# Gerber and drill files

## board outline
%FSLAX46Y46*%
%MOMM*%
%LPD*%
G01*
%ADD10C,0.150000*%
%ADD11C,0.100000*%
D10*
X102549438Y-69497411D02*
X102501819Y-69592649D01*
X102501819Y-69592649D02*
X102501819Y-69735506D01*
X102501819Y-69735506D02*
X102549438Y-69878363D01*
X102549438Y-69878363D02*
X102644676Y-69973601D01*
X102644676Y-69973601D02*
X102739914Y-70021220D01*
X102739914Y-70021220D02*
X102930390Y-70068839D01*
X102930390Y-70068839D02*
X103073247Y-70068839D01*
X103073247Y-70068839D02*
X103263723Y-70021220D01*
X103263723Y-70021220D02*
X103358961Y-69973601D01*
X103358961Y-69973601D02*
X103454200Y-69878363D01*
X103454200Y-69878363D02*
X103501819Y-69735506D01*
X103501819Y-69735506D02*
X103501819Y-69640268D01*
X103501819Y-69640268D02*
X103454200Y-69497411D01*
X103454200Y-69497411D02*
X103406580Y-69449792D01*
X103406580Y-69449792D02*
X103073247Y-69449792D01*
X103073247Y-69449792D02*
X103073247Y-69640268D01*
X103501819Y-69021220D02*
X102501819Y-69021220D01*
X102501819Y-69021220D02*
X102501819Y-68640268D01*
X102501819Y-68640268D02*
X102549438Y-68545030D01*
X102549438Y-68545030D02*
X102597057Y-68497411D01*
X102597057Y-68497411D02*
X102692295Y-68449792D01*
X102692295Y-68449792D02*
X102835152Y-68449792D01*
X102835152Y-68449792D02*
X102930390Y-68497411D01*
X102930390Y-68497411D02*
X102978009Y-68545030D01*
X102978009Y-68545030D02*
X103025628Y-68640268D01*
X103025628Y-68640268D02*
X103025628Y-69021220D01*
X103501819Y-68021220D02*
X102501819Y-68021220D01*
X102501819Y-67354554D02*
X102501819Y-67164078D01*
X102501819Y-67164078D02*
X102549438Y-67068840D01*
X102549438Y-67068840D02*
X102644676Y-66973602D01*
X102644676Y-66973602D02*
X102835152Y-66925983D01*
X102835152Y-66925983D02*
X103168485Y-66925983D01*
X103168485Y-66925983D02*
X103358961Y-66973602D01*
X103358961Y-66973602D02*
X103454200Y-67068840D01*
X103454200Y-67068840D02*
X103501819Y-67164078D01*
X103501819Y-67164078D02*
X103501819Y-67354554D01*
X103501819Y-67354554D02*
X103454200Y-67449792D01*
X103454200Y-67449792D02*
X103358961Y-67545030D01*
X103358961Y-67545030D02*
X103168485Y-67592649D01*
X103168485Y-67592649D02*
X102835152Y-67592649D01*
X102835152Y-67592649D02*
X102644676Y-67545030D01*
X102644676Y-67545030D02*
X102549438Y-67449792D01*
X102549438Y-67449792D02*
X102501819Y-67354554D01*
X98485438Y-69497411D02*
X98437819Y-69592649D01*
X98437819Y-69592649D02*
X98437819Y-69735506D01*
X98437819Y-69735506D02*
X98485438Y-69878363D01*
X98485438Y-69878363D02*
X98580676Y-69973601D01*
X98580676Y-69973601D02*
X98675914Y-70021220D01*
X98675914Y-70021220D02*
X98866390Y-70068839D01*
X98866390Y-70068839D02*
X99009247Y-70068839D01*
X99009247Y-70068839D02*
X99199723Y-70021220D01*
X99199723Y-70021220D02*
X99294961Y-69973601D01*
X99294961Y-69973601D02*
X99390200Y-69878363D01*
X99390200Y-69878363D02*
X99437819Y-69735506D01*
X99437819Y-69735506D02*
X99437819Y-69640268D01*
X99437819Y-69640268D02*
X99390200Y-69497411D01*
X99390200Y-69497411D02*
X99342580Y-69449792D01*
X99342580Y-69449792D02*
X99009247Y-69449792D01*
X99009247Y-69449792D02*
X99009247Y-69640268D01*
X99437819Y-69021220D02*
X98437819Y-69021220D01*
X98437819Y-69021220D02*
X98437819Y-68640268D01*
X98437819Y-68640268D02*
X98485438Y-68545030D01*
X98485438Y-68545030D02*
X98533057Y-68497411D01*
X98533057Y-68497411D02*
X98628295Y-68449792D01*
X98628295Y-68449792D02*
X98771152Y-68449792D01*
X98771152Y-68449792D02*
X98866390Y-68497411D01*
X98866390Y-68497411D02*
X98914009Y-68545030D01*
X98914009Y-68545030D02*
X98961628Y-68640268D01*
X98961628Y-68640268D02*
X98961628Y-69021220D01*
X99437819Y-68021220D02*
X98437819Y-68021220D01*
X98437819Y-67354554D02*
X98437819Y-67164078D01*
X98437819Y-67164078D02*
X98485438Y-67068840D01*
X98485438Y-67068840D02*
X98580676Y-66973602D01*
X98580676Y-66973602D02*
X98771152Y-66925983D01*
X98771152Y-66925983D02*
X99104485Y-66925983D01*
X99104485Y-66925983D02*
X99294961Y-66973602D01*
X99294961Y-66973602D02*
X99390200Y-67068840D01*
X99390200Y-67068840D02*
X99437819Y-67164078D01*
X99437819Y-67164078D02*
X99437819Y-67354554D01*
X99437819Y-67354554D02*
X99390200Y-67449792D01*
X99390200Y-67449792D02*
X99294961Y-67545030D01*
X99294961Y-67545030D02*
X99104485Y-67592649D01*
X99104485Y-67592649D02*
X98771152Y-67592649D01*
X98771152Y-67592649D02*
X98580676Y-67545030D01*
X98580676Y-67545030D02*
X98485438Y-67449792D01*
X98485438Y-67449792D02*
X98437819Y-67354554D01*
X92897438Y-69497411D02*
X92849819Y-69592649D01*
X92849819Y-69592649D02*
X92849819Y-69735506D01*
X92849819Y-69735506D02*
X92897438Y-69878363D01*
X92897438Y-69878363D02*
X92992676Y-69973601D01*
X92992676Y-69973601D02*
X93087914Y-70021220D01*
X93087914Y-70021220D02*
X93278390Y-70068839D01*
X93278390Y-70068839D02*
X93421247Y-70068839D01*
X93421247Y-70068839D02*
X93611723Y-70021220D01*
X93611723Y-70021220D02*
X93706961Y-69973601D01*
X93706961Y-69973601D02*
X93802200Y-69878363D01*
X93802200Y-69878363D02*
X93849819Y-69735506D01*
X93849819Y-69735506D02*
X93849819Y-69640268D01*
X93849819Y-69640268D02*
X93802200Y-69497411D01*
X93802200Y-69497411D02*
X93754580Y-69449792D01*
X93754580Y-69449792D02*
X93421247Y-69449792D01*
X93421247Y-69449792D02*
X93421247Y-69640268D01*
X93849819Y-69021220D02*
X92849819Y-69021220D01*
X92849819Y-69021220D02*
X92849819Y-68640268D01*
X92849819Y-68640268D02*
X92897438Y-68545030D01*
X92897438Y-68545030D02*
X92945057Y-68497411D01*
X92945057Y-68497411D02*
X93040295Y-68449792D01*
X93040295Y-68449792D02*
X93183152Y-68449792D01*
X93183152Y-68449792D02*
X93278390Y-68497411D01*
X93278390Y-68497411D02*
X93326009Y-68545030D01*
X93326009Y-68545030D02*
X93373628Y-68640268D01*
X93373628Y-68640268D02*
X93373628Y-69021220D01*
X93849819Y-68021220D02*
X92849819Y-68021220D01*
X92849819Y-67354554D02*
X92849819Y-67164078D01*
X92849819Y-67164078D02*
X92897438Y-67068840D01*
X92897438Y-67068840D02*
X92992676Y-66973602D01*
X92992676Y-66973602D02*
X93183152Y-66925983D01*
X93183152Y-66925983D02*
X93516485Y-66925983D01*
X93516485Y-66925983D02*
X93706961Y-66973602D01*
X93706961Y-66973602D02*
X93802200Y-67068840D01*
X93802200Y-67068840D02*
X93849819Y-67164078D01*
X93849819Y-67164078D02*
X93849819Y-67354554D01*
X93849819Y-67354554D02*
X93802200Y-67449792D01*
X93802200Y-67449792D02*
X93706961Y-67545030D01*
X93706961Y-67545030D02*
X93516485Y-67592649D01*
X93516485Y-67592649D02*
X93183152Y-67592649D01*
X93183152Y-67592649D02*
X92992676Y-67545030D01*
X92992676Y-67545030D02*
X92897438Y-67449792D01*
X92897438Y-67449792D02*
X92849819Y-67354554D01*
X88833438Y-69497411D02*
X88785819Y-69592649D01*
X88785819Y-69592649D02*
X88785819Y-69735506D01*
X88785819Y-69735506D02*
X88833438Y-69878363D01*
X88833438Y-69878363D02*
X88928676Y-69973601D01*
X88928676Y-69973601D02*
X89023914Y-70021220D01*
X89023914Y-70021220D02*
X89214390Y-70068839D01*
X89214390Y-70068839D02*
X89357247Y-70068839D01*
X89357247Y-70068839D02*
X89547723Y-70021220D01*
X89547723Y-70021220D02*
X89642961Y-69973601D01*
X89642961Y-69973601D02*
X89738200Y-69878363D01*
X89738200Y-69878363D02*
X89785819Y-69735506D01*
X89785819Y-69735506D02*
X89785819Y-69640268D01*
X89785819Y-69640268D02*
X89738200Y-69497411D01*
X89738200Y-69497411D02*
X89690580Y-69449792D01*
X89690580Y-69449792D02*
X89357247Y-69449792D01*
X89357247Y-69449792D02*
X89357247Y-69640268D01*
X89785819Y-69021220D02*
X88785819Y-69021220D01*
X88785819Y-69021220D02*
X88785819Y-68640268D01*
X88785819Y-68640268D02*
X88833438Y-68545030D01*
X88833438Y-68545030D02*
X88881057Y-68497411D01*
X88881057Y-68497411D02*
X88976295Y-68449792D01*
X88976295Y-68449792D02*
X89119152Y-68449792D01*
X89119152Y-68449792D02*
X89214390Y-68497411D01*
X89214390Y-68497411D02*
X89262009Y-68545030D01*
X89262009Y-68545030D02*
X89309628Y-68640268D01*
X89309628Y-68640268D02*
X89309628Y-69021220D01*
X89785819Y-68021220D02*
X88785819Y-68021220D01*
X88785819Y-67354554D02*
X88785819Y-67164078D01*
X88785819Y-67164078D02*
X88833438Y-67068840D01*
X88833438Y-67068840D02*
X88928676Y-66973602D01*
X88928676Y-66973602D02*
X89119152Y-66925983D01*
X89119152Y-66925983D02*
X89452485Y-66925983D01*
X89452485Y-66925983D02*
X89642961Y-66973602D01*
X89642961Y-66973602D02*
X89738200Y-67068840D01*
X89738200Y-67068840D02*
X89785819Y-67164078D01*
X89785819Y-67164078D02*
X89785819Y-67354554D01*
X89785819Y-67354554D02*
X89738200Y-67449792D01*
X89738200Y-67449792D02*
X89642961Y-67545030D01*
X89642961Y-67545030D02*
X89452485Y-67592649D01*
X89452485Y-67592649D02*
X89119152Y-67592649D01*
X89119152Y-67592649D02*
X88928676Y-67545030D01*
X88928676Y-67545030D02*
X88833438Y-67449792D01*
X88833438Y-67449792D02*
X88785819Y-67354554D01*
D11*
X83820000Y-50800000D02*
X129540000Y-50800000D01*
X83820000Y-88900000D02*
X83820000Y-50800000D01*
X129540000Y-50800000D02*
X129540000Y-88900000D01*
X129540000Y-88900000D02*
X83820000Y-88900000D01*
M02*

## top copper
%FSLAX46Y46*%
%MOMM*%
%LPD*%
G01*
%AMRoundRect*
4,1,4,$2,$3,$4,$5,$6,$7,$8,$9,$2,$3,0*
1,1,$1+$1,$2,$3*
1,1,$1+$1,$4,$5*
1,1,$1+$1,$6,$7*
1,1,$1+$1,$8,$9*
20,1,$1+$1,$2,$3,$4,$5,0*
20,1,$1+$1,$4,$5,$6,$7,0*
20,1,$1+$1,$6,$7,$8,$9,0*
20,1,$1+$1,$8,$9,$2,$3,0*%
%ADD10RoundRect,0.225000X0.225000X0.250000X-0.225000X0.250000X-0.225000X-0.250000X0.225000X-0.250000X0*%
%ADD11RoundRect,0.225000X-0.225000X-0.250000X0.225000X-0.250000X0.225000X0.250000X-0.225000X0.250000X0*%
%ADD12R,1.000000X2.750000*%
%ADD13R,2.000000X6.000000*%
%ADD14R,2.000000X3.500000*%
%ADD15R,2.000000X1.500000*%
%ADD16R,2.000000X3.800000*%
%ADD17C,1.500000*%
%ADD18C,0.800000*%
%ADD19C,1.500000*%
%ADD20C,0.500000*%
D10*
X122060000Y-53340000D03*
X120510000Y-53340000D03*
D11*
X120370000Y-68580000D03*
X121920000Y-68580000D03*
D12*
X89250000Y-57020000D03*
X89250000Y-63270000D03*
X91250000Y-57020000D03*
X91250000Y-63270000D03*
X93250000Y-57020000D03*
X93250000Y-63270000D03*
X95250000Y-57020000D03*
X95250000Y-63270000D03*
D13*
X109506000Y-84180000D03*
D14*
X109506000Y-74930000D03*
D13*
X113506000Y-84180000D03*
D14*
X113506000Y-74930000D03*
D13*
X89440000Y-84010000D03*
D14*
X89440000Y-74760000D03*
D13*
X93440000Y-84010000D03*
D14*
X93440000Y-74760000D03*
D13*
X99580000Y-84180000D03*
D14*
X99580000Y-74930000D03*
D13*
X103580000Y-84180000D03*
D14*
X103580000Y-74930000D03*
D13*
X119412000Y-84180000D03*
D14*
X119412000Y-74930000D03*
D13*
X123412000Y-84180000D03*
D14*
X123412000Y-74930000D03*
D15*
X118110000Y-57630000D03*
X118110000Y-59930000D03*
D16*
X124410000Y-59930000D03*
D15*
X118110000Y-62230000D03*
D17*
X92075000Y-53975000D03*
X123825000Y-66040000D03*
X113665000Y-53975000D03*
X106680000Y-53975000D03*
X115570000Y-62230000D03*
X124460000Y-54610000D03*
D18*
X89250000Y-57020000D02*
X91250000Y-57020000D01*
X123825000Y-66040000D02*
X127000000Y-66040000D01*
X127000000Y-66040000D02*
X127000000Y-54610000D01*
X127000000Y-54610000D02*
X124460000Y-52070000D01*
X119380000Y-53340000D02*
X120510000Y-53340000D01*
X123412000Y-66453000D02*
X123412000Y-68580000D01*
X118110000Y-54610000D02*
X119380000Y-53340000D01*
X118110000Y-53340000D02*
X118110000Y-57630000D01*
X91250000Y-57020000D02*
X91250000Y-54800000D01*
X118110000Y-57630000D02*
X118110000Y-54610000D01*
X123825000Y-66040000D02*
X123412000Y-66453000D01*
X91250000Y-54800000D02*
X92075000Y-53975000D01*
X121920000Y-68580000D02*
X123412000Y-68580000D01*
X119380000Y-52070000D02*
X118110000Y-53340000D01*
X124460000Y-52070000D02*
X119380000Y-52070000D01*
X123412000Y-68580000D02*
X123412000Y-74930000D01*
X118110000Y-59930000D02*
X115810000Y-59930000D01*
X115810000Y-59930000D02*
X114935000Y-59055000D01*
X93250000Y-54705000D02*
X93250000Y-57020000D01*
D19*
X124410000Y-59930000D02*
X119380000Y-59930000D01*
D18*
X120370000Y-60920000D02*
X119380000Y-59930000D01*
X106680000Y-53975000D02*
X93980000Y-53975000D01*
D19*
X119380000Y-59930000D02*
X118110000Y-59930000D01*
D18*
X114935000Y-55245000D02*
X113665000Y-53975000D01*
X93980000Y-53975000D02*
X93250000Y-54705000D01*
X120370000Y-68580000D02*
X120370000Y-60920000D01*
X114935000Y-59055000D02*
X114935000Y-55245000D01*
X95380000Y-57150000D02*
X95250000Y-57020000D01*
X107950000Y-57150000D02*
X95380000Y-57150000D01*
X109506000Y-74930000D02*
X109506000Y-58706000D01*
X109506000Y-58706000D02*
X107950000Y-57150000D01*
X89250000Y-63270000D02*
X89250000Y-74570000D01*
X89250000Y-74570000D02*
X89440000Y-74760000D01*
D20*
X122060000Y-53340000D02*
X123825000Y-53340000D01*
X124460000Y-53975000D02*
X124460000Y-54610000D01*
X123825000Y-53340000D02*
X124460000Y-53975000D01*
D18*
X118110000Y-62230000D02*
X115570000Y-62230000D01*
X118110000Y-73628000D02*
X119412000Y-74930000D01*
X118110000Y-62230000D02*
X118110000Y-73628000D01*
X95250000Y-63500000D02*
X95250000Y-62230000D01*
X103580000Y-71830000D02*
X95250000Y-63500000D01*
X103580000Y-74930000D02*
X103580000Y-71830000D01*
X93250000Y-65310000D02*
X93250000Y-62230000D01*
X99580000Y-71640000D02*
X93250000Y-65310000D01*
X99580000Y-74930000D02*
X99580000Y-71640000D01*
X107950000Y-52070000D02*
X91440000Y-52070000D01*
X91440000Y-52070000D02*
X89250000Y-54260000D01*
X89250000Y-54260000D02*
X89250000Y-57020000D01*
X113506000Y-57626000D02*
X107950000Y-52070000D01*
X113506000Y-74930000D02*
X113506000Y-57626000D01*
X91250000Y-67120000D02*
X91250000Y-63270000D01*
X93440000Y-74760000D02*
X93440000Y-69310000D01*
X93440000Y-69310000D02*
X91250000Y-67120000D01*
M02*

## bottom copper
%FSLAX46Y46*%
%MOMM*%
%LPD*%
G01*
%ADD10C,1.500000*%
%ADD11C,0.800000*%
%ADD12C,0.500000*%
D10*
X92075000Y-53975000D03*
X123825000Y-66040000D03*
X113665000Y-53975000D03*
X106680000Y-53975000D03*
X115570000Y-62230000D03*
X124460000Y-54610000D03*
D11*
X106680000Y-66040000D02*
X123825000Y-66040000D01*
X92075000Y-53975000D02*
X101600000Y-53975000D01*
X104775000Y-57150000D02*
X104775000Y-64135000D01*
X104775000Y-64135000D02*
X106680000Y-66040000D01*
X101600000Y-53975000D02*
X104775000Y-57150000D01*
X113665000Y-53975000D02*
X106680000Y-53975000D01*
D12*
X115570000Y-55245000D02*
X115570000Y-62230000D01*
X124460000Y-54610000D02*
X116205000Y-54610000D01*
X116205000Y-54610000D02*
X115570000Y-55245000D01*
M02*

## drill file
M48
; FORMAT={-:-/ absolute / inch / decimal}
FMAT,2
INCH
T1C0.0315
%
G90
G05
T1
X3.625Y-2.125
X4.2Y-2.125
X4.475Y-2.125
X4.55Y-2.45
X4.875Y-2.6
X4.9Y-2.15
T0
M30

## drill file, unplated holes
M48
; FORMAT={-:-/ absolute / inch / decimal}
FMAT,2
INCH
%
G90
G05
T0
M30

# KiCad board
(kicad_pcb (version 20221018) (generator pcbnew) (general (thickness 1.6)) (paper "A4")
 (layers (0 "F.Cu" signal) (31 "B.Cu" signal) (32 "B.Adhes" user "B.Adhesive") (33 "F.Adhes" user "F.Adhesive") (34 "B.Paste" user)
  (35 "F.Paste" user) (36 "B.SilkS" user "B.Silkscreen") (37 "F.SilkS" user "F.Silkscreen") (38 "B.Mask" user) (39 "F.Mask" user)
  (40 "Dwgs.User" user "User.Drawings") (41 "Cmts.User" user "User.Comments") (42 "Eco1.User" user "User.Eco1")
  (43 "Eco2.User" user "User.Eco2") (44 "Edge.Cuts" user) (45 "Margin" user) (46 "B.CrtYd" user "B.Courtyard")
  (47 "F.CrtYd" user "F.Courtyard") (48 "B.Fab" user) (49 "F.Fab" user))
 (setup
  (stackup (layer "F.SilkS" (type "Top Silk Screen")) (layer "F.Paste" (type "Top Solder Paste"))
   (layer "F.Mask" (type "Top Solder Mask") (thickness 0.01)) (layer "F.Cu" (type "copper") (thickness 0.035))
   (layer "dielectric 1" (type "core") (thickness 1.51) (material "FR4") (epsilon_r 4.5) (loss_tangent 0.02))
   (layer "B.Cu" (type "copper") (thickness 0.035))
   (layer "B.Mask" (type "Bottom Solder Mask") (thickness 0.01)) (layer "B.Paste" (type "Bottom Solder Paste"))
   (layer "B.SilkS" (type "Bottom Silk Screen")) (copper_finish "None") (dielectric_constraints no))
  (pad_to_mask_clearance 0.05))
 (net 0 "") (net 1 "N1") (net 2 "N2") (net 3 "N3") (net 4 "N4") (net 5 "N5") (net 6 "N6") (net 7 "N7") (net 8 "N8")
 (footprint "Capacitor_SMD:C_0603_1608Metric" (layer "F.Cu") (at 121.285 53.34 180)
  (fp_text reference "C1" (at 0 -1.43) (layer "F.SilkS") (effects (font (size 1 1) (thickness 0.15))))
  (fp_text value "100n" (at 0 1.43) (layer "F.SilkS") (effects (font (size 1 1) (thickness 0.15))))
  (pad "1" smd roundrect (at -0.775 0 180) (size 0.9 0.95) (layers "F.Cu" "F.Paste" "F.Mask") (roundrect_rratio 0.25) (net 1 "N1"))
  (pad "2" smd roundrect (at 0.775 0 180) (size 0.9 0.95) (layers "F.Cu" "F.Paste" "F.Mask") (roundrect_rratio 0.25) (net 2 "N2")))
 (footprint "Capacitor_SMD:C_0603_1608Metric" (layer "F.Cu") (at 121.145 68.58)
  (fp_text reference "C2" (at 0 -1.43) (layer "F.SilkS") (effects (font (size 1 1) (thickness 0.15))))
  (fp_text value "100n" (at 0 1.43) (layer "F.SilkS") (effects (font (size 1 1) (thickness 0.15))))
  (pad "1" smd roundrect (at -0.775 0) (size 0.9 0.95) (layers "F.Cu" "F.Paste" "F.Mask") (roundrect_rratio 0.25) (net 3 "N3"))
  (pad "2" smd roundrect (at 0.775 0) (size 0.9 0.95) (layers "F.Cu" "F.Paste" "F.Mask") (roundrect_rratio 0.25) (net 2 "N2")))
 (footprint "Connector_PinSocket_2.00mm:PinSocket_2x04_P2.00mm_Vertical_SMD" (layer "F.Cu") (at 92.25 60.145 90)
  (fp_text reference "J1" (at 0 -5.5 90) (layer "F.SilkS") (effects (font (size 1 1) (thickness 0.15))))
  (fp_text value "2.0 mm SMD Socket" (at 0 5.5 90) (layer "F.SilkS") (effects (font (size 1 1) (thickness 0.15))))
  (pad "1" smd rect (at 3.125 -3 90) (size 2.75 1) (layers "F.Cu" "F.Paste" "F.Mask") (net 2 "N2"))
  (pad "2" smd rect (at -3.125 -3 90) (size 2.75 1) (layers "F.Cu" "F.Paste" "F.Mask") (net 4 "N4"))
  (pad "3" smd rect (at 3.125 -1 90) (size 2.75 1) (layers "F.Cu" "F.Paste" "F.Mask") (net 2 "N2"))
  (pad "4" smd rect (at -3.125 -1 90) (size 2.75 1) (layers "F.Cu" "F.Paste" "F.Mask") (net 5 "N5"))
  (pad "5" smd rect (at 3.125 1 90) (size 2.75 1) (layers "F.Cu" "F.Paste" "F.Mask") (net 3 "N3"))
  (pad "6" smd rect (at -3.125 1 90) (size 2.75 1) (layers "F.Cu" "F.Paste" "F.Mask") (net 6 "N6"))
  (pad "7" smd rect (at 3.125 3 90) (size 2.75 1) (layers "F.Cu" "F.Paste" "F.Mask") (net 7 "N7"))
  (pad "8" smd rect (at -3.125 3 90) (size 2.75 1) (layers "F.Cu" "F.Paste" "F.Mask") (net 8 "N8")))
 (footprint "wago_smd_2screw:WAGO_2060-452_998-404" (layer "F.Cu") (at 111.506 80.18 90)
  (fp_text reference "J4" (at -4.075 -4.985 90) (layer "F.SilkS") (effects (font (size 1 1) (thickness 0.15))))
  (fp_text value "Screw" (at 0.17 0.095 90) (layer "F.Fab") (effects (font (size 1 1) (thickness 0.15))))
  (pad "1" smd rect (at -4 -2 90) (size 6 2) (layers "F.Cu" "F.Paste" "F.Mask") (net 7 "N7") (solder_mask_margin 0.102))
  (pad "1" smd rect (at 5.25 -2 90) (size 3.5 2) (layers "F.Cu" "F.Paste" "F.Mask") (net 7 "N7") (solder_mask_margin 0.102))
  (pad "2" smd rect (at -4 2 90) (size 6 2) (layers "F.Cu" "F.Paste" "F.Mask") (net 2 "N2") (solder_mask_margin 0.102))
  (pad "2" smd rect (at 5.25 2 90) (size 3.5 2) (layers "F.Cu" "F.Paste" "F.Mask") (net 2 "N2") (solder_mask_margin 0.102)))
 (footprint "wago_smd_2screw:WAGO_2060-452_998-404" (layer "F.Cu") (at 91.44 80.01 90)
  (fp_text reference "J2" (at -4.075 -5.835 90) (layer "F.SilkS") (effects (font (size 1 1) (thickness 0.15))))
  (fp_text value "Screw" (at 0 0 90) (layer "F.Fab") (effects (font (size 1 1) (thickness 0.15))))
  (pad "1" smd rect (at -4 -2 90) (size 6 2) (layers "F.Cu" "F.Paste" "F.Mask") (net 4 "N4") (solder_mask_margin 0.102))
  (pad "1" smd rect (at 5.25 -2 90) (size 3.5 2) (layers "F.Cu" "F.Paste" "F.Mask") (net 4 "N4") (solder_mask_margin 0.102))
  (pad "2" smd rect (at -4 2 90) (size 6 2) (layers "F.Cu" "F.Paste" "F.Mask") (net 5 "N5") (solder_mask_margin 0.102))
  (pad "2" smd rect (at 5.25 2 90) (size 3.5 2) (layers "F.Cu" "F.Paste" "F.Mask") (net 5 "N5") (solder_mask_margin 0.102)))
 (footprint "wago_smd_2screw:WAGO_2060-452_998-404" (layer "F.Cu") (at 101.58 80.18 90)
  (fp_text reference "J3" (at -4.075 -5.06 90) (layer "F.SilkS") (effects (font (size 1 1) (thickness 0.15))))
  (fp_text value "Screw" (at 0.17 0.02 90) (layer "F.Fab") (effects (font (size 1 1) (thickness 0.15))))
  (pad "1" smd rect (at -4 -2 90) (size 6 2) (layers "F.Cu" "F.Paste" "F.Mask") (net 6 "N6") (solder_mask_margin 0.102))
  (pad "1" smd rect (at 5.25 -2 90) (size 3.5 2) (layers "F.Cu" "F.Paste" "F.Mask") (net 6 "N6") (solder_mask_margin 0.102))
  (pad "2" smd rect (at -4 2 90) (size 6 2) (layers "F.Cu" "F.Paste" "F.Mask") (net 8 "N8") (solder_mask_margin 0.102))
  (pad "2" smd rect (at 5.25 2 90) (size 3.5 2) (layers "F.Cu" "F.Paste" "F.Mask") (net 8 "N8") (solder_mask_margin 0.102)))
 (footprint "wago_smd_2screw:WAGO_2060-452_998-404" (layer "F.Cu") (at 121.412 80.18 90)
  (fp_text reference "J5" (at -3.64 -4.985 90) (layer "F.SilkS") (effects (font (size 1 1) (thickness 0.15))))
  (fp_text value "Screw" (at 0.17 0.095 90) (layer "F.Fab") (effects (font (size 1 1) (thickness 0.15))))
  (pad "1" smd rect (at -4 -2 90) (size 6 2) (layers "F.Cu" "F.Paste" "F.Mask") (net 1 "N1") (solder_mask_margin 0.102))
  (pad "1" smd rect (at 5.25 -2 90) (size 3.5 2) (layers "F.Cu" "F.Paste" "F.Mask") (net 1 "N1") (solder_mask_margin 0.102))
  (pad "2" smd rect (at -4 2 90) (size 6 2) (layers "F.Cu" "F.Paste" "F.Mask") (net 2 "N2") (solder_mask_margin 0.102))
  (pad "2" smd rect (at 5.25 2 90) (size 3.5 2) (layers "F.Cu" "F.Paste" "F.Mask") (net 2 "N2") (solder_mask_margin 0.102)))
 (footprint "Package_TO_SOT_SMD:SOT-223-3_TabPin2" (layer "F.Cu") (at 121.26 59.93)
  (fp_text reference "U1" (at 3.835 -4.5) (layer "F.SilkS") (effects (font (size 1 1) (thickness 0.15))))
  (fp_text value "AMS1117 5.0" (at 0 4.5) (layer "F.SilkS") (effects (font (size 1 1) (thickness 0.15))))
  (pad "1" smd rect (at -3.15 -2.3) (size 2 1.5) (layers "F.Cu" "F.Paste" "F.Mask") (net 2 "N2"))
  (pad "2" smd rect (at -3.15 0) (size 2 1.5) (layers "F.Cu" "F.Paste" "F.Mask") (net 3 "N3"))
  (pad "2" smd rect (at 3.15 0) (size 2 3.8) (layers "F.Cu" "F.Paste" "F.Mask") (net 3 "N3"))
  (pad "3" smd rect (at -3.15 2.3) (size 2 1.5) (layers "F.Cu" "F.Paste" "F.Mask") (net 1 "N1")))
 (gr_line (start 83.82 50.8) (end 129.54 50.8) (stroke (width 0.1) (type default)) (layer "Edge.Cuts"))
 (gr_line (start 83.82 88.9) (end 83.82 50.8) (stroke (width 0.1) (type default)) (layer "Edge.Cuts"))
 (gr_line (start 129.54 50.8) (end 129.54 88.9) (stroke (width 0.1) (type default)) (layer "Edge.Cuts"))
 (gr_line (start 129.54 88.9) (end 83.82 88.9) (stroke (width 0.1) (type default)) (layer "Edge.Cuts"))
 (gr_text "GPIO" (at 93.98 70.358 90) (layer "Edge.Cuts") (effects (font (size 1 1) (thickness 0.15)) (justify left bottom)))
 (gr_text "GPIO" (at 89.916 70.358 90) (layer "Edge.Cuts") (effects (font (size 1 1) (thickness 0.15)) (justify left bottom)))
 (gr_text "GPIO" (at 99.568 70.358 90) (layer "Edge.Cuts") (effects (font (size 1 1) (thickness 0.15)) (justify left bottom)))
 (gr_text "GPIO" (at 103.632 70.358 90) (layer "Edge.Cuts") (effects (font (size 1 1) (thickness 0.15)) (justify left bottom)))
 (segment (start 118.11 59.93) (end 115.81 59.93) (width 0.8) (layer "F.Cu") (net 3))
 (segment (start 115.81 59.93) (end 114.935 59.055) (width 0.8) (layer "F.Cu") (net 3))
 (segment (start 93.25 54.705) (end 93.25 57.02) (width 0.8) (layer "F.Cu") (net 3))
 (segment (start 124.41 59.93) (end 119.38 59.93) (width 1.5) (layer "F.Cu") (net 3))
 (segment (start 120.37 60.92) (end 119.38 59.93) (width 0.8) (layer "F.Cu") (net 3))
 (segment (start 106.68 53.975) (end 93.98 53.975) (width 0.8) (layer "F.Cu") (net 3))
 (segment (start 119.38 59.93) (end 118.11 59.93) (width 1.5) (layer "F.Cu") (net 3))
 (segment (start 114.935 55.245) (end 113.665 53.975) (width 0.8) (layer "F.Cu") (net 3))
 (segment (start 93.98 53.975) (end 93.25 54.705) (width 0.8) (layer "F.Cu") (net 3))
 (segment (start 120.37 68.58) (end 120.37 60.92) (width 0.8) (layer "F.Cu") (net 3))
 (segment (start 114.935 59.055) (end 114.935 55.245) (width 0.8) (layer "F.Cu") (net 3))
 (via (at 113.665 53.975) (size 1.5) (drill 0.8) (layers "F.Cu" "B.Cu") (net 3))
 (via (at 106.68 53.975) (size 1.5) (drill 0.8) (layers "F.Cu" "B.Cu") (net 3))
 (segment (start 113.665 53.975) (end 106.68 53.975) (width 0.8) (layer "B.Cu") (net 3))
 (segment (start 95.38 57.15) (end 95.25 57.02) (width 0.8) (layer "F.Cu") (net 7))
 (segment (start 107.95 57.15) (end 95.38 57.15) (width 0.8) (layer "F.Cu") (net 7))
 (segment (start 109.506 74.93) (end 109.506 58.706) (width 0.8) (layer "F.Cu") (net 7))
 (segment (start 109.506 58.706) (end 107.95 57.15) (width 0.8) (layer "F.Cu") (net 7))
 (segment (start 89.25 63.27) (end 89.25 74.57) (width 0.8) (layer "F.Cu") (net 4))
 (segment (start 89.25 74.57) (end 89.44 74.76) (width 0.8) (layer "F.Cu") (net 4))
 (segment (start 122.06 53.34) (end 123.825 53.34) (width 0.5) (layer "F.Cu") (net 1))
 (segment (start 124.46 53.975) (end 124.46 54.61) (width 0.5) (layer "F.Cu") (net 1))
 (segment (start 123.825 53.34) (end 124.46 53.975) (width 0.5) (layer "F.Cu") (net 1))
 (segment (start 118.11 62.23) (end 115.57 62.23) (width 0.8) (layer "F.Cu") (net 1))
 (segment (start 118.11 73.628) (end 119.412 74.93) (width 0.8) (layer "F.Cu") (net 1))
 (segment (start 118.11 62.23) (end 118.11 73.628) (width 0.8) (layer "F.Cu") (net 1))
 (via (at 115.57 62.23) (size 1.5) (drill 0.8) (layers "F.Cu" "B.Cu") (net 1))
 (via (at 124.46 54.61) (size 1.5) (drill 0.8) (layers "F.Cu" "B.Cu") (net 1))
 (segment (start 115.57 55.245) (end 115.57 62.23) (width 0.5) (layer "B.Cu") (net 1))
 (segment (start 124.46 54.61) (end 116.205 54.61) (width 0.5) (layer "B.Cu") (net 1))
 (segment (start 116.205 54.61) (end 115.57 55.245) (width 0.5) (layer "B.Cu") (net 1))
 (segment (start 95.25 63.5) (end 95.25 62.23) (width 0.8) (layer "F.Cu") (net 8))
 (segment (start 103.58 71.83) (end 95.25 63.5) (width 0.8) (layer "F.Cu") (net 8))
 (segment (start 103.58 74.93) (end 103.58 71.83) (width 0.8) (layer "F.Cu") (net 8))
 (segment (start 93.25 65.31) (end 93.25 62.23) (width 0.8) (layer "F.Cu") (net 6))
 (segment (start 99.58 71.64) (end 93.25 65.31) (width 0.8) (layer "F.Cu") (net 6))
 (segment (start 99.58 74.93) (end 99.58 71.64) (width 0.8) (layer "F.Cu") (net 6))
 (segment (start 123.825 66.04) (end 127 66.04) (width 0.8) (layer "F.Cu") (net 2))
 (segment (start 127 66.04) (end 127 54.61) (width 0.8) (layer "F.Cu") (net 2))
 (segment (start 107.95 52.07) (end 91.44 52.07) (width 0.8) (layer "F.Cu") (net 2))
 (segment (start 127 54.61) (end 124.46 52.07) (width 0.8) (layer "F.Cu") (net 2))
 (segment (start 91.44 52.07) (end 89.25 54.26) (width 0.8) (layer "F.Cu") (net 2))
 (segment (start 89.25 54.26) (end 89.25 57.02) (width 0.8) (layer "F.Cu") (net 2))
 (segment (start 119.38 53.34) (end 120.51 53.34) (width 0.8) (layer "F.Cu") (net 2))
 (segment (start 123.412 66.453) (end 123.412 68.58) (width 0.8) (layer "F.Cu") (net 2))
 (segment (start 113.506 57.626) (end 107.95 52.07) (width 0.8) (layer "F.Cu") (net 2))
 (segment (start 118.11 54.61) (end 119.38 53.34) (width 0.8) (layer "F.Cu") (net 2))
 (segment (start 118.11 53.34) (end 118.11 57.63) (width 0.8) (layer "F.Cu") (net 2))
 (segment (start 91.25 57.02) (end 91.25 54.8) (width 0.8) (layer "F.Cu") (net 2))
 (segment (start 118.11 57.63) (end 118.11 54.61) (width 0.8) (layer "F.Cu") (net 2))
 (segment (start 123.825 66.04) (end 123.412 66.453) (width 0.8) (layer "F.Cu") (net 2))
 (segment (start 91.25 54.8) (end 92.075 53.975) (width 0.8) (layer "F.Cu") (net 2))
 (segment (start 89.25 57.02) (end 91.25 57.02) (width 0.8) (layer "F.Cu") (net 2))
 (segment (start 121.92 68.58) (end 123.412 68.58) (width 0.8) (layer "F.Cu") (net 2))
 (segment (start 113.506 74.93) (end 113.506 57.626) (width 0.8) (layer "F.Cu") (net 2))
 (segment (start 119.38 52.07) (end 118.11 53.34) (width 0.8) (layer "F.Cu") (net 2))
 (segment (start 124.46 52.07) (end 119.38 52.07) (width 0.8) (layer "F.Cu") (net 2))
 (segment (start 123.412 68.58) (end 123.412 74.93) (width 0.8) (layer "F.Cu") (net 2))
 (via (at 92.075 53.975) (size 1.5) (drill 0.8) (layers "F.Cu" "B.Cu") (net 2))
 (via (at 123.825 66.04) (size 1.5) (drill 0.8) (layers "F.Cu" "B.Cu") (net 2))
 (segment (start 106.68 66.04) (end 123.825 66.04) (width 0.8) (layer "B.Cu") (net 2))
 (segment (start 92.075 53.975) (end 101.6 53.975) (width 0.8) (layer "B.Cu") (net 2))
 (segment (start 104.775 57.15) (end 104.775 64.135) (width 0.8) (layer "B.Cu") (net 2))
 (segment (start 104.775 64.135) (end 106.68 66.04) (width 0.8) (layer "B.Cu") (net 2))
 (segment (start 101.6 53.975) (end 104.775 57.15) (width 0.8) (layer "B.Cu") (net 2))
 (segment (start 91.25 67.12) (end 91.25 63.27) (width 0.8) (layer "F.Cu") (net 5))
 (segment (start 93.44 74.76) (end 93.44 69.31) (width 0.8) (layer "F.Cu") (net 5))
 (segment (start 93.44 69.31) (end 91.25 67.12) (width 0.8) (layer "F.Cu") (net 5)))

